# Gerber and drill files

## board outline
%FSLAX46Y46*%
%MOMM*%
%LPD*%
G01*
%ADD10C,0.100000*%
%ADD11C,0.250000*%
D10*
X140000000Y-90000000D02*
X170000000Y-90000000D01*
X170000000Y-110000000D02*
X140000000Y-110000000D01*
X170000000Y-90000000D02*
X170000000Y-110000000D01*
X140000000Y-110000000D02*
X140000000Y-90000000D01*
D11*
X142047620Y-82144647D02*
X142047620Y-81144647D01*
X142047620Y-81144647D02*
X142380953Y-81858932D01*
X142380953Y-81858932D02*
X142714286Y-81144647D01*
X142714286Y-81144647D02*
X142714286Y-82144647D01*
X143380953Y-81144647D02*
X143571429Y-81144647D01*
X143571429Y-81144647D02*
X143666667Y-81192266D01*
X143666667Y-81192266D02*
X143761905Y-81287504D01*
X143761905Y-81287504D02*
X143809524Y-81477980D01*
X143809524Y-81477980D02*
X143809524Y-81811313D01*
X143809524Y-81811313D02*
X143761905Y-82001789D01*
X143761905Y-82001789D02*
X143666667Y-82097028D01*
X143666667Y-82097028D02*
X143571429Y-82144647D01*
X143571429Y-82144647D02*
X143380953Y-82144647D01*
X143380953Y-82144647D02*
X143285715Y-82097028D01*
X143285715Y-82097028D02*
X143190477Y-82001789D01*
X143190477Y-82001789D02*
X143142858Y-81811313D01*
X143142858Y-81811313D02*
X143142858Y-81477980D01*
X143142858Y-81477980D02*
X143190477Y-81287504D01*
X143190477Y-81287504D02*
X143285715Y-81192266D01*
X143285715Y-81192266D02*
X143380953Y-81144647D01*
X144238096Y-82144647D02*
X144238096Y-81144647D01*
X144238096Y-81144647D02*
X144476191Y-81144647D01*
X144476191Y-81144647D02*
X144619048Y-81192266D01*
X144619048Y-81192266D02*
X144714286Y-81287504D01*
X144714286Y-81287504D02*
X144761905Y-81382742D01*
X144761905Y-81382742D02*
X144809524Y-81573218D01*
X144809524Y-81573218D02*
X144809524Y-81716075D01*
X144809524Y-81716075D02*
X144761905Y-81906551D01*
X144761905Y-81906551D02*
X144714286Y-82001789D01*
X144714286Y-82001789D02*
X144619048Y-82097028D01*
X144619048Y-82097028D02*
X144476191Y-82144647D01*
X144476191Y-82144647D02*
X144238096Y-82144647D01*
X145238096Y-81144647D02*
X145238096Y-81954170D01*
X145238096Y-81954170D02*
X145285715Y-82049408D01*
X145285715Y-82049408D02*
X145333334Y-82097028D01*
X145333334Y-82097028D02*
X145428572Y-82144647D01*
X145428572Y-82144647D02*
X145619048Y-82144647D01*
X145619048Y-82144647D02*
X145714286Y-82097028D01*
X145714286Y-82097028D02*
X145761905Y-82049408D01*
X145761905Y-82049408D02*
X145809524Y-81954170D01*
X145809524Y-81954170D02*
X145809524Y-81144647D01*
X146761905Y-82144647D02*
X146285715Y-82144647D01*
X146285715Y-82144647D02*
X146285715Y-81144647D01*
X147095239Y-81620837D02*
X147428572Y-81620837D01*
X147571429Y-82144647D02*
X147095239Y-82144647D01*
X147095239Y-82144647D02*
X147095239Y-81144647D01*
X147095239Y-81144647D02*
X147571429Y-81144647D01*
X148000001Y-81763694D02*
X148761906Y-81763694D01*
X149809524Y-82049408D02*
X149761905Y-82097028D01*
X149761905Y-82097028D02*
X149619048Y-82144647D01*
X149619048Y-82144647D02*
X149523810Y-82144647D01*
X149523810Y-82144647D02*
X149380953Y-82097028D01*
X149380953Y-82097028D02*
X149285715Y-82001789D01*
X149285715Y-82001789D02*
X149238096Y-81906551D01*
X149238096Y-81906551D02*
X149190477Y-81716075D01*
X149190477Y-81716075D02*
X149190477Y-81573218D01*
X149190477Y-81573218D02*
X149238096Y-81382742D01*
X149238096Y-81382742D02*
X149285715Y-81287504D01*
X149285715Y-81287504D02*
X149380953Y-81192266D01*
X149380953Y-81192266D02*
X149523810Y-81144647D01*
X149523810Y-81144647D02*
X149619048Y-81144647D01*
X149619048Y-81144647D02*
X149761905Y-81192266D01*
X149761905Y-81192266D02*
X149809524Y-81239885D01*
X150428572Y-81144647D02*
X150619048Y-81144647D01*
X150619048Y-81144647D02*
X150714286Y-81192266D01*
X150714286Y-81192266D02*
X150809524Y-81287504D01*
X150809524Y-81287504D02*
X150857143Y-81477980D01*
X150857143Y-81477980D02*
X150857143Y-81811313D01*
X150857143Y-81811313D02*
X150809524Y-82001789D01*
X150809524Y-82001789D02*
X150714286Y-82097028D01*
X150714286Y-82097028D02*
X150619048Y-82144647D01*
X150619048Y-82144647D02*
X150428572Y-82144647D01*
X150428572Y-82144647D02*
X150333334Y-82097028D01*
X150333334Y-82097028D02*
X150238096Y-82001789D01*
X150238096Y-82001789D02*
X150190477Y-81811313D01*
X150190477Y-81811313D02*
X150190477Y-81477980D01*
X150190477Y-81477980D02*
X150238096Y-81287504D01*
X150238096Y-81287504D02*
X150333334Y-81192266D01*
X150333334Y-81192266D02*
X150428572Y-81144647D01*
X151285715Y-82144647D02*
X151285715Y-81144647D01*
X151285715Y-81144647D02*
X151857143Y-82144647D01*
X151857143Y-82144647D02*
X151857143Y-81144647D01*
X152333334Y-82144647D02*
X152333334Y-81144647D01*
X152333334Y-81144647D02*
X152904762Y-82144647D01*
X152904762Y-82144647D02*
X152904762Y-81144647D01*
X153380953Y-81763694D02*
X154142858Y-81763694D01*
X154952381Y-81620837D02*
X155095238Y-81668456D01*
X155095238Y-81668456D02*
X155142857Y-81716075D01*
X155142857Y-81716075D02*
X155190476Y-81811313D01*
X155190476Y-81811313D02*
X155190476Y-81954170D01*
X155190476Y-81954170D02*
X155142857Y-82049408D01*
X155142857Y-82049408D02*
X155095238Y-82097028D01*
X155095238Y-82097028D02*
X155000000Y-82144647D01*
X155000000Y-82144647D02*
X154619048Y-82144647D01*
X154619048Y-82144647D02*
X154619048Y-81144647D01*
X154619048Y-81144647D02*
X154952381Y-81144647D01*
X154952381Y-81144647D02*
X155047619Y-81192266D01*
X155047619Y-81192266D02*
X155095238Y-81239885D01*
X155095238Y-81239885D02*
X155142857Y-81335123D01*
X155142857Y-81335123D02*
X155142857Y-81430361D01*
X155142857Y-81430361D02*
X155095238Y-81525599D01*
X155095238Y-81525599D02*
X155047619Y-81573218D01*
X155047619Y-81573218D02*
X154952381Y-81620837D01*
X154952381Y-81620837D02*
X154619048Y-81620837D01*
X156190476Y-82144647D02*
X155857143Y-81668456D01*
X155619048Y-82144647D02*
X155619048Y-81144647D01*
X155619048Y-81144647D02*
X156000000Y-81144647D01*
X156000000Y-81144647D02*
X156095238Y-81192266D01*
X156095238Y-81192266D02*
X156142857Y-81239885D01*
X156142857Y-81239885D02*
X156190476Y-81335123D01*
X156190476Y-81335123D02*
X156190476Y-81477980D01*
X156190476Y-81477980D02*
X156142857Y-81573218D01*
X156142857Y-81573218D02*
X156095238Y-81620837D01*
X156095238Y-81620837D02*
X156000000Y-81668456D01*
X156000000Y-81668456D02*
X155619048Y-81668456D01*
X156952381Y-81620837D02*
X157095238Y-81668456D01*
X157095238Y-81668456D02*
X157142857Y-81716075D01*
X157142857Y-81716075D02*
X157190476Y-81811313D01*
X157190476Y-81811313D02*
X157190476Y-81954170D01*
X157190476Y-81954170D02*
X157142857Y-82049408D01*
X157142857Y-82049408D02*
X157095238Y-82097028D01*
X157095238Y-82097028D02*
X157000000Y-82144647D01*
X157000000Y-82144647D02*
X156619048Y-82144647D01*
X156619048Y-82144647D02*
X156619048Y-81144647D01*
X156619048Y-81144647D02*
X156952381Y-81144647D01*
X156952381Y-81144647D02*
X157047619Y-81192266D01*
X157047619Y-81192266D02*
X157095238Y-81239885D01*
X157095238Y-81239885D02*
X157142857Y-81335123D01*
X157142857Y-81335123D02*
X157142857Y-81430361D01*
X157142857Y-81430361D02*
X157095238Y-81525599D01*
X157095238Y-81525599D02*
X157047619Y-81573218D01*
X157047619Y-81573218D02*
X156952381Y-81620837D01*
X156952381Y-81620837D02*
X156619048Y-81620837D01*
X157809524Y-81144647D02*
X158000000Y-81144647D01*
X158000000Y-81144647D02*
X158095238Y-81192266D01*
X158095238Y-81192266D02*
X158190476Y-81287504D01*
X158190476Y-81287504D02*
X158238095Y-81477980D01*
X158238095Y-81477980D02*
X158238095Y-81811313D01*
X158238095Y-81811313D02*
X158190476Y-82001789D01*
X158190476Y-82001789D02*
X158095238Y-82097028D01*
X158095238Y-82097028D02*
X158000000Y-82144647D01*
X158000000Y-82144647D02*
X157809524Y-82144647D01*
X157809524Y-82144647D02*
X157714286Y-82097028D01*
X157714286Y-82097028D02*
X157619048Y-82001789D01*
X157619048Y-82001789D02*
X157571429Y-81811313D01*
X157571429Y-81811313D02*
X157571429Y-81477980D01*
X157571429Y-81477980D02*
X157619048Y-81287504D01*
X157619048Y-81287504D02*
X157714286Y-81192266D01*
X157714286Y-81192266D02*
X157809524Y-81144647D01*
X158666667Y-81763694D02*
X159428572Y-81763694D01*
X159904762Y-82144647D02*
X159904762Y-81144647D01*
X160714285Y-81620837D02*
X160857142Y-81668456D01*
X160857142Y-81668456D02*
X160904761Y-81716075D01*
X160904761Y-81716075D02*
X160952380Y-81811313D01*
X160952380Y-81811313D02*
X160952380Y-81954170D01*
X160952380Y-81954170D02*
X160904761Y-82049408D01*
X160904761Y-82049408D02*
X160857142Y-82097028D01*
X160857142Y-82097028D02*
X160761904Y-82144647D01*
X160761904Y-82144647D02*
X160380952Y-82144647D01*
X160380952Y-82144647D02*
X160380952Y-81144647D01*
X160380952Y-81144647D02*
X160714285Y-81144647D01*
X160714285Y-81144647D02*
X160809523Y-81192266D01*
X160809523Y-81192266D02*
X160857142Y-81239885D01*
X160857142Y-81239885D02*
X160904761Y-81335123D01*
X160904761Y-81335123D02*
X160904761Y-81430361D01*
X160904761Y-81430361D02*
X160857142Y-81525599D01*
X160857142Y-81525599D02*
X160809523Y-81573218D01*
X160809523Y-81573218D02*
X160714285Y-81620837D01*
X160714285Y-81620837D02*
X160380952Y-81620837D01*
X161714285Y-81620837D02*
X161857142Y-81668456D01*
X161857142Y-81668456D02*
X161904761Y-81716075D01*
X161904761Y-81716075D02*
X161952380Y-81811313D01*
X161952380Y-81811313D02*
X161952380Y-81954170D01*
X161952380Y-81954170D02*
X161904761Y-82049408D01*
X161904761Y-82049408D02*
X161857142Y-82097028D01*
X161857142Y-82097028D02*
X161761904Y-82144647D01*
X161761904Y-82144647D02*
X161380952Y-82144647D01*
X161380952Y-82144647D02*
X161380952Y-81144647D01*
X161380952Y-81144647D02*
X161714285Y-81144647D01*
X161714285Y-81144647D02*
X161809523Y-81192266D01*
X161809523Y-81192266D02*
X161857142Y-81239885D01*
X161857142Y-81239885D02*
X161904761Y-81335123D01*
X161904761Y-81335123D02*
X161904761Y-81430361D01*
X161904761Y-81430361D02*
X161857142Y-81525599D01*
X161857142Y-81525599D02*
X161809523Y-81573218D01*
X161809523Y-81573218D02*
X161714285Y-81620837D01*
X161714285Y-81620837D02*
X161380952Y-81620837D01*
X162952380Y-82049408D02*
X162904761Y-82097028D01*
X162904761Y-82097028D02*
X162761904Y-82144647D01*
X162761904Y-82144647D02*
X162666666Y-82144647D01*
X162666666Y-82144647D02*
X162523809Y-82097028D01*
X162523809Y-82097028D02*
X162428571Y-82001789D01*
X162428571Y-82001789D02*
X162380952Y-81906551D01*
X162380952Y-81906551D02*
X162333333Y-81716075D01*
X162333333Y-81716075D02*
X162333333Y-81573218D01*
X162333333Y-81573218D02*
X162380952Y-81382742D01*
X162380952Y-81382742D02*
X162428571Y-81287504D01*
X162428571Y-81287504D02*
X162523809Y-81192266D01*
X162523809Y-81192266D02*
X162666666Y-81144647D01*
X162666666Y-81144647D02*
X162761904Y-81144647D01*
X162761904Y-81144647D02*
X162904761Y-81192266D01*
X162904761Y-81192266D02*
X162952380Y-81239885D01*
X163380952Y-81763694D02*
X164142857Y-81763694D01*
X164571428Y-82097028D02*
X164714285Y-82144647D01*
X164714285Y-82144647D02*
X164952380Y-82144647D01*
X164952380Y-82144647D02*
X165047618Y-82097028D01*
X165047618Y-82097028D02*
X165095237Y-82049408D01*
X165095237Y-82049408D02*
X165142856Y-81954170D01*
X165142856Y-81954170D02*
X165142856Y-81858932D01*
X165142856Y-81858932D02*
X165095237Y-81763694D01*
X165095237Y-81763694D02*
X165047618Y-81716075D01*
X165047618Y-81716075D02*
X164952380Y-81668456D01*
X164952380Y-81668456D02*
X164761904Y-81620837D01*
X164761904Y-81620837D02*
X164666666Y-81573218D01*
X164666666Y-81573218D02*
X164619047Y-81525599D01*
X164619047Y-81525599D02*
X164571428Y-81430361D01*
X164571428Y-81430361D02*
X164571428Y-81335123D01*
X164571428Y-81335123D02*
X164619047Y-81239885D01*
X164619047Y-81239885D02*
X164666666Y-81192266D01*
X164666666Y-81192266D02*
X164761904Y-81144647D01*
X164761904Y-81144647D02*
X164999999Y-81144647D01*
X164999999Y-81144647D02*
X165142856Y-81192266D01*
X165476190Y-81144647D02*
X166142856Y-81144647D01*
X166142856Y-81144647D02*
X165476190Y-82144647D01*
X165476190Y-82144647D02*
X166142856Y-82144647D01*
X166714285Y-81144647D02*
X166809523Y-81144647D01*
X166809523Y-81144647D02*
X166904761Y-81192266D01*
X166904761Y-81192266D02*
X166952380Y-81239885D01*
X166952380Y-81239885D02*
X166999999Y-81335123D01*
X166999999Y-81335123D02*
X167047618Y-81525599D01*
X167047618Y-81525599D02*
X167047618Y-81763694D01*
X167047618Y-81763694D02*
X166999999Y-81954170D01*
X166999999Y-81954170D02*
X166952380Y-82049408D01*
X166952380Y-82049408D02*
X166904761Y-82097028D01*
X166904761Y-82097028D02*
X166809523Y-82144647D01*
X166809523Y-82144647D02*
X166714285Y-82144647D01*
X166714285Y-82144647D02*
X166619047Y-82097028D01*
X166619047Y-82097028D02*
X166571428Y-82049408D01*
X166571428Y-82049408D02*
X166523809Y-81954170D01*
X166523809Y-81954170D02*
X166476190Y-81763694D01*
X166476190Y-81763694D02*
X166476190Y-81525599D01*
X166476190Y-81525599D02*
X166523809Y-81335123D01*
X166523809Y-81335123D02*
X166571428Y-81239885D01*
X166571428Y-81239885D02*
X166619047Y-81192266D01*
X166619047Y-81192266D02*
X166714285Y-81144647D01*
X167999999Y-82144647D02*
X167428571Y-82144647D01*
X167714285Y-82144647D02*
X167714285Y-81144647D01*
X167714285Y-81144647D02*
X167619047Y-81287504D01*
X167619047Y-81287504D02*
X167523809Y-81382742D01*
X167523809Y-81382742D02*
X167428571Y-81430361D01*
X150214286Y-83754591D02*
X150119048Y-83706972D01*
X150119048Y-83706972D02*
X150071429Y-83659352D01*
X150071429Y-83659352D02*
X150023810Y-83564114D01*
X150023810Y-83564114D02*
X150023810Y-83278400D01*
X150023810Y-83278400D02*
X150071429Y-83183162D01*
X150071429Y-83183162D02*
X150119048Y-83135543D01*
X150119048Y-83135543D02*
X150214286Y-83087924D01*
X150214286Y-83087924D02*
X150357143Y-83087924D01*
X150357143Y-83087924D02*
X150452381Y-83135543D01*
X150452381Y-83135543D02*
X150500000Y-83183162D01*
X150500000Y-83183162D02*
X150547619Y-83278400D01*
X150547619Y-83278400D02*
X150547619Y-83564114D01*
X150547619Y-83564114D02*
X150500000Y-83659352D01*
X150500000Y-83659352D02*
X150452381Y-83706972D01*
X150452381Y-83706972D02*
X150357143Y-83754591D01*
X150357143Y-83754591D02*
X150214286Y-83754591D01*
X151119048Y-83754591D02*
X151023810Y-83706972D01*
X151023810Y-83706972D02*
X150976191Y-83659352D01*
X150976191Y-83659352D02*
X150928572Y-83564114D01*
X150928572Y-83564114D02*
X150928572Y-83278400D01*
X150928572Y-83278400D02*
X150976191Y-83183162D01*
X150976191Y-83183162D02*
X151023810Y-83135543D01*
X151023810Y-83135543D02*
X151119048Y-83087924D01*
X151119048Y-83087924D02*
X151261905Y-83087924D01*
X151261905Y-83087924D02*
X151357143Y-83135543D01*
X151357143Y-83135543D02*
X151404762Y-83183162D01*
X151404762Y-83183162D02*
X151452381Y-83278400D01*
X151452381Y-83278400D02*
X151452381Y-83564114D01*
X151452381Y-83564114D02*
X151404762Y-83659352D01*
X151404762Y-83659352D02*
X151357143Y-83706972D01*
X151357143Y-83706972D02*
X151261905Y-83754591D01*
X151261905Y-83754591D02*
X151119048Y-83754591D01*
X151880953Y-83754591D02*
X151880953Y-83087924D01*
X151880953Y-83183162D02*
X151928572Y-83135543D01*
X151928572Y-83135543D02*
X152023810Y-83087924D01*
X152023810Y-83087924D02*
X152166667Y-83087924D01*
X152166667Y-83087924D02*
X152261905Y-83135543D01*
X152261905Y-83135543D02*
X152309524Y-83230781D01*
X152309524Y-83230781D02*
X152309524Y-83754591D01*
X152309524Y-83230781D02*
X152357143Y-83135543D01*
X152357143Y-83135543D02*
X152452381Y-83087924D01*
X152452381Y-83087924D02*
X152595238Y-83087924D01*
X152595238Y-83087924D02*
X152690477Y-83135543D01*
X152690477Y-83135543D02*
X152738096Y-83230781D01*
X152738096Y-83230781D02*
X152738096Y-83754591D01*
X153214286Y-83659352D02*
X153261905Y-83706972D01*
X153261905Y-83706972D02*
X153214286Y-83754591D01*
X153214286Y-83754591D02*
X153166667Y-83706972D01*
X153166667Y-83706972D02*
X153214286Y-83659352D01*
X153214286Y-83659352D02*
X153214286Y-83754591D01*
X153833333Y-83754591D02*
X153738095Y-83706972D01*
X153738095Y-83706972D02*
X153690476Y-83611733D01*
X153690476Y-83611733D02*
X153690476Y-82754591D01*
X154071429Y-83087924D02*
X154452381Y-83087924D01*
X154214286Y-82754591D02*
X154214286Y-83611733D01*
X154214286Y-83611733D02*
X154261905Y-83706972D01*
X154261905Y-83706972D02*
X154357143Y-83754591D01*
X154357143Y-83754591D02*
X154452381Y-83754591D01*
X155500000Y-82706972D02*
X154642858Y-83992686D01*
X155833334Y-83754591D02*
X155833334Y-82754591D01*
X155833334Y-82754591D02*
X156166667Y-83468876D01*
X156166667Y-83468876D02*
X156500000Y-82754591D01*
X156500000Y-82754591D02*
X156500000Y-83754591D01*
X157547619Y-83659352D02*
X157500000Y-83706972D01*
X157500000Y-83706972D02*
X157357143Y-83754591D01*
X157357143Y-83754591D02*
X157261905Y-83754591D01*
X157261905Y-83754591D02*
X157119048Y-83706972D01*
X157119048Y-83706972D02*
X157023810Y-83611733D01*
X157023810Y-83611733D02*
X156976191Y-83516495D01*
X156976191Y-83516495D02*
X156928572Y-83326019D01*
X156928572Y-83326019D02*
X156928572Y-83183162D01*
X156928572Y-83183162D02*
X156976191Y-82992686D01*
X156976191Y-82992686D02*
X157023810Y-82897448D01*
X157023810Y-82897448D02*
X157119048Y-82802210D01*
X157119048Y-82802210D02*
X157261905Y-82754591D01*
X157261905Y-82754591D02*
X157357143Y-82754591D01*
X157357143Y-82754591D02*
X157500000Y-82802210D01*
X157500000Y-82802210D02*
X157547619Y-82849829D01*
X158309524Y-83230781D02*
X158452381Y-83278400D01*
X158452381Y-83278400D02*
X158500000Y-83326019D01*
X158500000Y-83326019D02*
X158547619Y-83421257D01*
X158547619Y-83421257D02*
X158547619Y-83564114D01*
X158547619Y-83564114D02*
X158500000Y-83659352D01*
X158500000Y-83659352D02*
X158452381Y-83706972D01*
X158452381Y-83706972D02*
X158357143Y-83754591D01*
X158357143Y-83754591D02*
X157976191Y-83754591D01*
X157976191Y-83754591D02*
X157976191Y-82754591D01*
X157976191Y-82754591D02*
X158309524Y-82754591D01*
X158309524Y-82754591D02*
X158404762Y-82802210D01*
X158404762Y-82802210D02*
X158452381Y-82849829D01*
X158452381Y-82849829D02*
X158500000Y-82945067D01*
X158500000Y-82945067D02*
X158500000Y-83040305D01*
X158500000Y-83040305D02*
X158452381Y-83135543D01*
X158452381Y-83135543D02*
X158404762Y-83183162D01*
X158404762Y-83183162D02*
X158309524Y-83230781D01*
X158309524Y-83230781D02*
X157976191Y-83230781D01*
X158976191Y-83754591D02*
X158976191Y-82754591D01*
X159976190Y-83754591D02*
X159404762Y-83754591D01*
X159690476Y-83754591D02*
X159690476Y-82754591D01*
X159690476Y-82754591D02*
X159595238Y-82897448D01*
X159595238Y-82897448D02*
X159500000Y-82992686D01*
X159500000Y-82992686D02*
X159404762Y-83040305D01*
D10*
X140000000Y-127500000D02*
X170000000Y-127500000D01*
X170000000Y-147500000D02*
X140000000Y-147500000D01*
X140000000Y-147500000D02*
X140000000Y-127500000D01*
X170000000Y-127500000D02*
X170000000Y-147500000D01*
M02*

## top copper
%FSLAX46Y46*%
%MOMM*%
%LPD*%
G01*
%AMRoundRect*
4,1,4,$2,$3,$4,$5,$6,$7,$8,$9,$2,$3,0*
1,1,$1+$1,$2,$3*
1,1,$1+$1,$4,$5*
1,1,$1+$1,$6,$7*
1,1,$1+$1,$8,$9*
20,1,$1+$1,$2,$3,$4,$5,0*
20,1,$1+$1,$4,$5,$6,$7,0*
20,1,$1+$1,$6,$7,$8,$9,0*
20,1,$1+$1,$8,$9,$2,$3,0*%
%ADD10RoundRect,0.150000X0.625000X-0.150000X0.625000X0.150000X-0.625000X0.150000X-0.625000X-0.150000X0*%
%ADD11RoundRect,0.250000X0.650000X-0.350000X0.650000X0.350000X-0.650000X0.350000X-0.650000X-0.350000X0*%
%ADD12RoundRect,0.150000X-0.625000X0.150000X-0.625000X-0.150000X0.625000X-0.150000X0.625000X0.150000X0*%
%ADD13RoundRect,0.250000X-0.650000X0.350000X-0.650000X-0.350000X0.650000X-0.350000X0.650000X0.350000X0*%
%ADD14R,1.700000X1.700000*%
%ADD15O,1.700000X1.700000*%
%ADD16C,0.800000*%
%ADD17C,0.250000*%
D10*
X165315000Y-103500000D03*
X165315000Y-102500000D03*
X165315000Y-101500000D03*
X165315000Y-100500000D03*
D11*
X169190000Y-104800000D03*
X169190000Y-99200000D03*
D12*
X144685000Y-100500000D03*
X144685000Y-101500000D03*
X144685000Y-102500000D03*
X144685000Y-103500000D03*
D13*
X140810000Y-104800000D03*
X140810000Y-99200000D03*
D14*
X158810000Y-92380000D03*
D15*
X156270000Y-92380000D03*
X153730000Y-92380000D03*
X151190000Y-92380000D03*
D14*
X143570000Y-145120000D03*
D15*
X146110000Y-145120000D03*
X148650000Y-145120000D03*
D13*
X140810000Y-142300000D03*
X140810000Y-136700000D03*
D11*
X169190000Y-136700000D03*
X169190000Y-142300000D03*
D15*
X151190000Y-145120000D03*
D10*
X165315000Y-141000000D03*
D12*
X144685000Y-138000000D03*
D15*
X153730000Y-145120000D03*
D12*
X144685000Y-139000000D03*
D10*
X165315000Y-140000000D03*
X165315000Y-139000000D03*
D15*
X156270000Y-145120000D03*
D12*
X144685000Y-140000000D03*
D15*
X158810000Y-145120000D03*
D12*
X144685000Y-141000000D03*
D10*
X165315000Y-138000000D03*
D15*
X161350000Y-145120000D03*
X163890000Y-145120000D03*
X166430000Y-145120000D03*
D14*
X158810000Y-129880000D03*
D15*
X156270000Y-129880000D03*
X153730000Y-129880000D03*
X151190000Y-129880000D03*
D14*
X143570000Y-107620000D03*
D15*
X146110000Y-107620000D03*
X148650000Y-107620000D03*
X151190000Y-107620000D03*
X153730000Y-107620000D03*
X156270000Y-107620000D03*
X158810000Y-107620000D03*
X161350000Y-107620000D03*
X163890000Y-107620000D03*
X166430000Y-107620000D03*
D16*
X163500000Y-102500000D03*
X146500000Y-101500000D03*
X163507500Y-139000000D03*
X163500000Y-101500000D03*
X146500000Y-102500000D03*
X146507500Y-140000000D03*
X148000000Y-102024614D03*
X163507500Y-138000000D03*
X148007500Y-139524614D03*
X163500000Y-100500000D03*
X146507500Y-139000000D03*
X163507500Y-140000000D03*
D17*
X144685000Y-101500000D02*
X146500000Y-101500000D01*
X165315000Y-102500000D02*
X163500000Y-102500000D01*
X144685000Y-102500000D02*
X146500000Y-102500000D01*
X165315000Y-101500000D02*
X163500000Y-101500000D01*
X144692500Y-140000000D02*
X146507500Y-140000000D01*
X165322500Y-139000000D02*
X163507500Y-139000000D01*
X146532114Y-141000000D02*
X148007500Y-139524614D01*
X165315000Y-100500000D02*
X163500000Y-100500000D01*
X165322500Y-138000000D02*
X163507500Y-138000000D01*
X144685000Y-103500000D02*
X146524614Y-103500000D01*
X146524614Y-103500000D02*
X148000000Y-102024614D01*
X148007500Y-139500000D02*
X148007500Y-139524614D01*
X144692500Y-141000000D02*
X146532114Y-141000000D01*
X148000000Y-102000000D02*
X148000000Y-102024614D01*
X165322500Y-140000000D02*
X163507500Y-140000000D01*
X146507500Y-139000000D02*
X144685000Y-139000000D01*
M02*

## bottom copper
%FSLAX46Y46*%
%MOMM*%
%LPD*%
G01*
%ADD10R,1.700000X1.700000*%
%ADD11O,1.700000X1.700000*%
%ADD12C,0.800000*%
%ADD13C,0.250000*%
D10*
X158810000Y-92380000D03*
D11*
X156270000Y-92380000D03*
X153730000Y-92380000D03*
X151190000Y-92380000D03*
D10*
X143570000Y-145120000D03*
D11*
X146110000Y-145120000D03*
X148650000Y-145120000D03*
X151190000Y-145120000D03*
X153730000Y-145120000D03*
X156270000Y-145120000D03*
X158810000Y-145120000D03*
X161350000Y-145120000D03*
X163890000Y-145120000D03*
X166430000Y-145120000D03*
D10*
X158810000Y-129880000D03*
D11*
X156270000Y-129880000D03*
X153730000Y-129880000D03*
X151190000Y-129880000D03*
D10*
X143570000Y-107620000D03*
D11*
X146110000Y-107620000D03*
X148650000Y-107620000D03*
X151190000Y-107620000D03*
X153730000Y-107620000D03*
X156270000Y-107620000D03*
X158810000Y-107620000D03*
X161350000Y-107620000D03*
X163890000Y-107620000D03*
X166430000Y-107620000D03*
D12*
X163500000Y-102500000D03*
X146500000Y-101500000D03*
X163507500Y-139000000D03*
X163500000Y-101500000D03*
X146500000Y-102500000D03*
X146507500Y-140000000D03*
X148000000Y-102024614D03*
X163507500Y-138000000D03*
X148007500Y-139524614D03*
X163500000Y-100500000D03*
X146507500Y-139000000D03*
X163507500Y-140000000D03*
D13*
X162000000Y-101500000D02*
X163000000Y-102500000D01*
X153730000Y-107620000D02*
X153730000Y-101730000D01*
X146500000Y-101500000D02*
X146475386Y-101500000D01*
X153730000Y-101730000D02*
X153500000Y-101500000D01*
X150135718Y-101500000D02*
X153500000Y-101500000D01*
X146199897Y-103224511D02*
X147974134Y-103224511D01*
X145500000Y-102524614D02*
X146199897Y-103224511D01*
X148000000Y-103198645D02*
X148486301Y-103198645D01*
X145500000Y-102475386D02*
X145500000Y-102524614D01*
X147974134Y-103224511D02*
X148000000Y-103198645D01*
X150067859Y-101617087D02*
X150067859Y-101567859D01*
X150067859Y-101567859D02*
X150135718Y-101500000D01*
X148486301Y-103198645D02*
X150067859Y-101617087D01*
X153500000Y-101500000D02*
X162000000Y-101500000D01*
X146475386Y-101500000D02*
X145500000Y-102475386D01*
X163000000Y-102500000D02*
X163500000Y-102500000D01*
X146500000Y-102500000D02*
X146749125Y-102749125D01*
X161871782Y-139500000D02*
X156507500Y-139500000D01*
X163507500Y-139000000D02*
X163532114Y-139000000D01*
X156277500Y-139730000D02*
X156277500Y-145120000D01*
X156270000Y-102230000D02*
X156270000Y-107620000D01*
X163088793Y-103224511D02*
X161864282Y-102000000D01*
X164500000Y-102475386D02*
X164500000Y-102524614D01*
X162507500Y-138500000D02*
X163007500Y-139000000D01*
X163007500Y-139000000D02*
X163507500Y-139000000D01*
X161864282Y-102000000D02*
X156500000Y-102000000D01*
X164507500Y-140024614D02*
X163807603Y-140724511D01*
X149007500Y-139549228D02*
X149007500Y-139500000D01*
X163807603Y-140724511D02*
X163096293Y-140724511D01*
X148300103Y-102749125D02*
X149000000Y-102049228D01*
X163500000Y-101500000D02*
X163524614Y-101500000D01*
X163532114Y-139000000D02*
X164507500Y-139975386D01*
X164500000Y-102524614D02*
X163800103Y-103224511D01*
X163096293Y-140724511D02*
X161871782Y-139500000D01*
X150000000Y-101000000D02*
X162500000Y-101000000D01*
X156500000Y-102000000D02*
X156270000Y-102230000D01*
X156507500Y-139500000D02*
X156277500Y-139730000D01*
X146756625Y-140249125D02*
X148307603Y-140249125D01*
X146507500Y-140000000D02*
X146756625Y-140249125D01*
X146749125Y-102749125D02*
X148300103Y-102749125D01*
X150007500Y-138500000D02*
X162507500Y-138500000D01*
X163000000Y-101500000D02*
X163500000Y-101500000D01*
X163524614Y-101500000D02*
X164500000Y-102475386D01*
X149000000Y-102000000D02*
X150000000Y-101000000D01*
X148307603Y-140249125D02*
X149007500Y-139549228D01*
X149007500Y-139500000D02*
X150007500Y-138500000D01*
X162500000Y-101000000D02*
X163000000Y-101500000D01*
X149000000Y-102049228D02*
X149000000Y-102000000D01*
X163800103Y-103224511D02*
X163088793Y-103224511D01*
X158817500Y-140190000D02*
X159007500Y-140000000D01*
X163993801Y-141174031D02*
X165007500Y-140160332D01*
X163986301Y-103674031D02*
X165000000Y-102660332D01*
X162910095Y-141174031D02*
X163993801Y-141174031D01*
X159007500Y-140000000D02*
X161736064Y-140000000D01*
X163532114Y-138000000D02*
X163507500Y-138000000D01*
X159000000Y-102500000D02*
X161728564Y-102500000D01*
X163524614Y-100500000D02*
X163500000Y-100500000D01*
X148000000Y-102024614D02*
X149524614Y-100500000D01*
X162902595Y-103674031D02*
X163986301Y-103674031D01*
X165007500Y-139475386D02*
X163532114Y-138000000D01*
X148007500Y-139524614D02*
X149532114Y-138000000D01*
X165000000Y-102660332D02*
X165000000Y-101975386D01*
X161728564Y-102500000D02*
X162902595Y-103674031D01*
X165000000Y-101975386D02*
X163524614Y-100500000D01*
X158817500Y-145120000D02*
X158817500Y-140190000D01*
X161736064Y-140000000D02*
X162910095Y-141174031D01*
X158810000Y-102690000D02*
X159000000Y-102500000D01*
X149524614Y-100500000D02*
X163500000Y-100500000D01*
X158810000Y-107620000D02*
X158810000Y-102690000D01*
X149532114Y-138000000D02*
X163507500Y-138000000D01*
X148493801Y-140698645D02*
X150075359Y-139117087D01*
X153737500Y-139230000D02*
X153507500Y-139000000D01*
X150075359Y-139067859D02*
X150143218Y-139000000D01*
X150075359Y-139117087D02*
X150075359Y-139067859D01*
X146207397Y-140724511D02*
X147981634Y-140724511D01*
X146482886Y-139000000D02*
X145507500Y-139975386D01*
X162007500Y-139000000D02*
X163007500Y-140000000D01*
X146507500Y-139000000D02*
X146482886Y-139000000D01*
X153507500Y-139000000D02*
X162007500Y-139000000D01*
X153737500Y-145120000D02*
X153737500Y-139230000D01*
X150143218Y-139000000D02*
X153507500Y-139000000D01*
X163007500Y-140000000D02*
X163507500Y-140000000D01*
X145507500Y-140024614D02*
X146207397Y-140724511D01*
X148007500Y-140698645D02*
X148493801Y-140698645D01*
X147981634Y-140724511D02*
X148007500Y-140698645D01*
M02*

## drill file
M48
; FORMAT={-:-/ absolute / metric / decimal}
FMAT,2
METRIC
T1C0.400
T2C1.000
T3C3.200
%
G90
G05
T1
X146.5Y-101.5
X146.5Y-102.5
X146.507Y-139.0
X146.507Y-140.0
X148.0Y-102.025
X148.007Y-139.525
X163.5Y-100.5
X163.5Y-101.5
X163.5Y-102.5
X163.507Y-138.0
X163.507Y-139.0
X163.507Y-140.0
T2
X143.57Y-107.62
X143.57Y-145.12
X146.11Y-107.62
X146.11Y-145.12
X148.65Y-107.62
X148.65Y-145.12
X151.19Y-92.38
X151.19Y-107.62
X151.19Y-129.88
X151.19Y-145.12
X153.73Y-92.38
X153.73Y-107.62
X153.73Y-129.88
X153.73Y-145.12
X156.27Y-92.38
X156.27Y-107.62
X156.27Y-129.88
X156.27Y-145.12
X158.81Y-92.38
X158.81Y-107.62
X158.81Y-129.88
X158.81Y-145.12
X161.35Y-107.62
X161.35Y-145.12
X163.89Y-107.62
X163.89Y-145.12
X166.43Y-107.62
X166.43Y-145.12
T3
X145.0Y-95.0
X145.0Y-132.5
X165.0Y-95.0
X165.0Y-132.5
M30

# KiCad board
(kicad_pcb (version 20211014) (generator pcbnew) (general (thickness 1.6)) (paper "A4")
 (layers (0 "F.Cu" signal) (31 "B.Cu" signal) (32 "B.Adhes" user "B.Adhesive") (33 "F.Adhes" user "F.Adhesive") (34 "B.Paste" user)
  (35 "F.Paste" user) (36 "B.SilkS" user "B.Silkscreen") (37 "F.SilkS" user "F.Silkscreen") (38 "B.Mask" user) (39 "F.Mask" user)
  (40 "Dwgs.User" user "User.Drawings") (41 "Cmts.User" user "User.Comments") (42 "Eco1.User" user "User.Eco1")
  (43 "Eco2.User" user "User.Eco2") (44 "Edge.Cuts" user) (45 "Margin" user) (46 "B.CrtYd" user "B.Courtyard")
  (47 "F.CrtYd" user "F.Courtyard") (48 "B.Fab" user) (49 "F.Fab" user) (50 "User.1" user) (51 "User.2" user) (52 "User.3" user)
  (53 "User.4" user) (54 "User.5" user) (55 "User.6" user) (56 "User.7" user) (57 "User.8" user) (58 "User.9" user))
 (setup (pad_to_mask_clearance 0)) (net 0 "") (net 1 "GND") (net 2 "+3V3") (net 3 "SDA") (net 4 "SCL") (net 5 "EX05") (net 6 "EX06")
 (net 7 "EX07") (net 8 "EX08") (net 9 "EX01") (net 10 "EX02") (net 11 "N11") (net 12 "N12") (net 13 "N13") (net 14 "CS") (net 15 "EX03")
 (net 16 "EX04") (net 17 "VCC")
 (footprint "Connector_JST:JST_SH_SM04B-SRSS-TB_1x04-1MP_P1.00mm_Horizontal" (layer "F.Cu") (at 167.315 102 90)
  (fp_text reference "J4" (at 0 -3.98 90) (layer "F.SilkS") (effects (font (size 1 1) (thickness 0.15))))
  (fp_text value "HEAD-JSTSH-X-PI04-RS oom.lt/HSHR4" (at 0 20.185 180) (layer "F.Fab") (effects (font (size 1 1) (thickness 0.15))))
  (pad "1" smd roundrect (at -1.5 -2 90) (size 0.6 1.55) (layers "F.Cu" "F.Paste" "F.Mask") (roundrect_rratio 0.25) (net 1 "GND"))
  (pad "2" smd roundrect (at -0.5 -2 90) (size 0.6 1.55) (layers "F.Cu" "F.Paste" "F.Mask") (roundrect_rratio 0.25) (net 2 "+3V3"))
  (pad "3" smd roundrect (at 0.5 -2 90) (size 0.6 1.55) (layers "F.Cu" "F.Paste" "F.Mask") (roundrect_rratio 0.25) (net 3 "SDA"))
  (pad "4" smd roundrect (at 1.5 -2 90) (size 0.6 1.55) (layers "F.Cu" "F.Paste" "F.Mask") (roundrect_rratio 0.25) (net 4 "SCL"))
  (pad "MP" smd roundrect (at -2.8 1.875 90) (size 1.2 1.8) (layers "F.Cu" "F.Paste" "F.Mask") (roundrect_rratio 0.208333) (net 1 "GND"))
  (pad "MP" smd roundrect (at 2.8 1.875 90) (size 1.2 1.8) (layers "F.Cu" "F.Paste" "F.Mask") (roundrect_rratio 0.208333) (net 1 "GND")))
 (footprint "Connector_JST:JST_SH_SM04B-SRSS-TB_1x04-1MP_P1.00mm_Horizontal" (layer "F.Cu") (at 142.685 102 -90)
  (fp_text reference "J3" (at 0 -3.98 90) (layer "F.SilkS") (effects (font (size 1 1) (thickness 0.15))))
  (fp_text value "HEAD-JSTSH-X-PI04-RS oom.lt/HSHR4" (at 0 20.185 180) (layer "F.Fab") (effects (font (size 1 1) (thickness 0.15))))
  (pad "1" smd roundrect (at -1.5 -2 270) (size 0.6 1.55) (layers "F.Cu" "F.Paste" "F.Mask") (roundrect_rratio 0.25) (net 1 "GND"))
  (pad "2" smd roundrect (at -0.5 -2 270) (size 0.6 1.55) (layers "F.Cu" "F.Paste" "F.Mask") (roundrect_rratio 0.25) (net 2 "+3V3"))
  (pad "3" smd roundrect (at 0.5 -2 270) (size 0.6 1.55) (layers "F.Cu" "F.Paste" "F.Mask") (roundrect_rratio 0.25) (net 3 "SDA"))
  (pad "4" smd roundrect (at 1.5 -2 270) (size 0.6 1.55) (layers "F.Cu" "F.Paste" "F.Mask") (roundrect_rratio 0.25) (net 4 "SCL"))
  (pad "MP" smd roundrect (at 2.8 1.875 270) (size 1.2 1.8) (layers "F.Cu" "F.Paste" "F.Mask") (roundrect_rratio 0.208333) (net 1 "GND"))
  (pad "MP" smd roundrect (at -2.8 1.875 270) (size 1.2 1.8) (layers "F.Cu" "F.Paste" "F.Mask") (roundrect_rratio 0.208333) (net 1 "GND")))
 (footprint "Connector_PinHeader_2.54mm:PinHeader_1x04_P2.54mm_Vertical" (layer "F.Cu") (at 158.81 92.38 -90)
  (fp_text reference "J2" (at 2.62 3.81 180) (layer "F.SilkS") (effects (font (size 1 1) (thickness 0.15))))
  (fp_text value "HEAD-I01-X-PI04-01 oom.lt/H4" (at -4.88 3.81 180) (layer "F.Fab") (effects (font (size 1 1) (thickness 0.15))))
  (pad "1" thru_hole rect (at 0 0 270) (size 1.7 1.7) (drill 1) (layers *.Cu *.Mask) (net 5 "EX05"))
  (pad "2" thru_hole oval (at 0 2.54 270) (size 1.7 1.7) (drill 1) (layers *.Cu *.Mask) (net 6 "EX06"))
  (pad "3" thru_hole oval (at 0 5.08 270) (size 1.7 1.7) (drill 1) (layers *.Cu *.Mask) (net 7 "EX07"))
  (pad "4" thru_hole oval (at 0 7.62 270) (size 1.7 1.7) (drill 1) (layers *.Cu *.Mask) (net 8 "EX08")))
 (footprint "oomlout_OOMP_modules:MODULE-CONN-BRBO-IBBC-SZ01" (layer "F.Cu") (at 155 137.5)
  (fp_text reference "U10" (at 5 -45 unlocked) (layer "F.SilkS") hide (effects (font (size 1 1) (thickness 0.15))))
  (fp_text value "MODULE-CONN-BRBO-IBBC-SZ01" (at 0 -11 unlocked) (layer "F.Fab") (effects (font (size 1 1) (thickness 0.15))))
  (fp_line (start -15 -10) (end 15 -10) (layer "Edge.Cuts") (width 0.1))
  (fp_line (start 15 10) (end -15 10) (layer "Edge.Cuts") (width 0.1))
  (fp_line (start -15 10) (end -15 -10) (layer "Edge.Cuts") (width 0.1))
  (fp_line (start 15 -10) (end 15 10) (layer "Edge.Cuts") (width 0.1))
  (pad "" np_thru_hole circle (at 10 -5) (size 3.2 3.2) (drill 3.2) (layers *.Cu *.Mask))
  (pad "" np_thru_hole circle (at -10 -5) (size 3.2 3.2) (drill 3.2) (layers *.Cu *.Mask))
  (pad "1" thru_hole rect (at -11.43 7.62 90) (size 1.7 1.7) (drill 1) (layers *.Cu *.Mask) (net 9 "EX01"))
  (pad "2" thru_hole oval (at -8.89 7.62 90) (size 1.7 1.7) (drill 1) (layers *.Cu *.Mask) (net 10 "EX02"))
  (pad "3" thru_hole oval (at -6.35 7.62 90) (size 1.7 1.7) (drill 1) (layers *.Cu *.Mask) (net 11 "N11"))
  (pad "4" smd roundrect (at -14.19 4.8 270) (size 1.2 1.8) (layers "F.Cu" "F.Paste" "F.Mask") (roundrect_rratio 0.208333) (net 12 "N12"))
  (pad "4" smd roundrect (at -14.19 -0.8 270) (size 1.2 1.8) (layers "F.Cu" "F.Paste" "F.Mask") (roundrect_rratio 0.208333) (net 12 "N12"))
  (pad "4" smd roundrect (at 14.19 -0.8 90) (size 1.2 1.8) (layers "F.Cu" "F.Paste" "F.Mask") (roundrect_rratio 0.208333) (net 12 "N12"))
  (pad "4" smd roundrect (at 14.19 4.8 90) (size 1.2 1.8) (layers "F.Cu" "F.Paste" "F.Mask") (roundrect_rratio 0.208333) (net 12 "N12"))
  (pad "4" thru_hole oval (at -3.81 7.62 90) (size 1.7 1.7) (drill 1) (layers *.Cu *.Mask) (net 12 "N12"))
  (pad "4" smd roundrect (at 10.315 3.5 90) (size 0.6 1.55) (layers "F.Cu" "F.Paste" "F.Mask") (roundrect_rratio 0.25) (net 12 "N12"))
  (pad "4" smd roundrect (at -10.315 0.5 270) (size 0.6 1.55) (layers "F.Cu" "F.Paste" "F.Mask") (roundrect_rratio 0.25) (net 12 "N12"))
  (pad "5" thru_hole oval (at -1.27 7.62 90) (size 1.7 1.7) (drill 1) (layers *.Cu *.Mask) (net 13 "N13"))
  (pad "5" smd roundrect (at -10.315 1.5 270) (size 0.6 1.55) (layers "F.Cu" "F.Paste" "F.Mask") (roundrect_rratio 0.25) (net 13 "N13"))
  (pad "5" smd roundrect (at 10.315 2.5 90) (size 0.6 1.55) (layers "F.Cu" "F.Paste" "F.Mask") (roundrect_rratio 0.25) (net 13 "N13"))
  (pad "6" smd roundrect (at 10.315 1.5 90) (size 0.6 1.55) (layers "F.Cu" "F.Paste" "F.Mask") (roundrect_rratio 0.25) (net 3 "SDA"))
  (pad "6" thru_hole oval (at 1.27 7.62 90) (size 1.7 1.7) (drill 1) (layers *.Cu *.Mask) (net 3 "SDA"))
  (pad "6" smd roundrect (at -10.315 2.5 270) (size 0.6 1.55) (layers "F.Cu" "F.Paste" "F.Mask") (roundrect_rratio 0.25) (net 3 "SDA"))
  (pad "7" thru_hole oval (at 3.81 7.62 90) (size 1.7 1.7) (drill 1) (layers *.Cu *.Mask) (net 4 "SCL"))
  (pad "7" smd roundrect (at -10.315 3.5 270) (size 0.6 1.55) (layers "F.Cu" "F.Paste" "F.Mask") (roundrect_rratio 0.25) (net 4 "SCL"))
  (pad "7" smd roundrect (at 10.315 0.5 90) (size 0.6 1.55) (layers "F.Cu" "F.Paste" "F.Mask") (roundrect_rratio 0.25) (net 4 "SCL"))
  (pad "8" thru_hole oval (at 6.35 7.62 90) (size 1.7 1.7) (drill 1) (layers *.Cu *.Mask) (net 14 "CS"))
  (pad "9" thru_hole oval (at 8.89 7.62 90) (size 1.7 1.7) (drill 1) (layers *.Cu *.Mask) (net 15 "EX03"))
  (pad "10" thru_hole oval (at 11.43 7.62 90) (size 1.7 1.7) (drill 1) (layers *.Cu *.Mask) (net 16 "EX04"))
  (pad "11" thru_hole rect (at 3.81 -7.62 270) (size 1.7 1.7) (drill 1) (layers *.Cu *.Mask) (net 5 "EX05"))
  (pad "12" thru_hole oval (at 1.27 -7.62 270) (size 1.7 1.7) (drill 1) (layers *.Cu *.Mask) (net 6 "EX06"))
  (pad "13" thru_hole oval (at -1.27 -7.62 270) (size 1.7 1.7) (drill 1) (layers *.Cu *.Mask) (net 7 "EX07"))
  (pad "14" thru_hole oval (at -3.81 -7.62 270) (size 1.7 1.7) (drill 1) (layers *.Cu *.Mask) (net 8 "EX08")))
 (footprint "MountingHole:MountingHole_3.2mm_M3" (layer "F.Cu") (at 145 95)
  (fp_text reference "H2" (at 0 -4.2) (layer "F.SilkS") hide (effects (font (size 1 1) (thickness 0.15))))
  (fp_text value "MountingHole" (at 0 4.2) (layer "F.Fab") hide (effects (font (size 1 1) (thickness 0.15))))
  (pad "" np_thru_hole circle (at 0 0) (size 3.2 3.2) (drill 3.2) (layers *.Cu *.Mask)))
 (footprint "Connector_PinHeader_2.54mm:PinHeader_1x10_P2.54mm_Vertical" (layer "F.Cu") (at 143.57 107.62 90)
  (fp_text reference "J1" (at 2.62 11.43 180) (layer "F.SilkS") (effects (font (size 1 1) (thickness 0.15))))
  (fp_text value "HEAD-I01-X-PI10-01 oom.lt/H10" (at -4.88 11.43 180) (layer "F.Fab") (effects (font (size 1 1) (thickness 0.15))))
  (pad "1" thru_hole rect (at 0 0 90) (size 1.7 1.7) (drill 1) (layers *.Cu *.Mask) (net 9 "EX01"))
  (pad "2" thru_hole oval (at 0 2.54 90) (size 1.7 1.7) (drill 1) (layers *.Cu *.Mask) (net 10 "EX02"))
  (pad "3" thru_hole oval (at 0 5.08 90) (size 1.7 1.7) (drill 1) (layers *.Cu *.Mask) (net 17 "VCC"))
  (pad "4" thru_hole oval (at 0 7.62 90) (size 1.7 1.7) (drill 1) (layers *.Cu *.Mask) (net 1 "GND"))
  (pad "5" thru_hole oval (at 0 10.16 90) (size 1.7 1.7) (drill 1) (layers *.Cu *.Mask) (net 2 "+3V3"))
  (pad "6" thru_hole oval (at 0 12.7 90) (size 1.7 1.7) (drill 1) (layers *.Cu *.Mask) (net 3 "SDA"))
  (pad "7" thru_hole oval (at 0 15.24 90) (size 1.7 1.7) (drill 1) (layers *.Cu *.Mask) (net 4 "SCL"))
  (pad "8" thru_hole oval (at 0 17.78 90) (size 1.7 1.7) (drill 1) (layers *.Cu *.Mask) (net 14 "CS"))
  (pad "9" thru_hole oval (at 0 20.32 90) (size 1.7 1.7) (drill 1) (layers *.Cu *.Mask) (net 15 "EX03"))
  (pad "10" thru_hole oval (at 0 22.86 90) (size 1.7 1.7) (drill 1) (layers *.Cu *.Mask) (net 16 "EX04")))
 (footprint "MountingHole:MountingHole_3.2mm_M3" (layer "F.Cu") (at 165 95)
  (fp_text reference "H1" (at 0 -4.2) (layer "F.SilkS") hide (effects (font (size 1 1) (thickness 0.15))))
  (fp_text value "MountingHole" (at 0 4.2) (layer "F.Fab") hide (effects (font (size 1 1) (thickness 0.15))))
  (pad "" np_thru_hole circle (at 0 0) (size 3.2 3.2) (drill 3.2) (layers *.Cu *.Mask)))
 (gr_line (start 140 90) (end 170 90) (layer "Edge.Cuts") (width 0.1))
 (gr_line (start 170 110) (end 140 110) (layer "Edge.Cuts") (width 0.1))
 (gr_line (start 170 90) (end 170 110) (layer "Edge.Cuts") (width 0.1))
 (gr_line (start 140 110) (end 140 90) (layer "Edge.Cuts") (width 0.1))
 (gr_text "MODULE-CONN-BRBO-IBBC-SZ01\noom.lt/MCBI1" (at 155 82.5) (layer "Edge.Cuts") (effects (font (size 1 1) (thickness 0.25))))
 (segment (start 144.685 101.5) (end 146.5 101.5) (width 0.25) (layer "F.Cu") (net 2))
 (segment (start 165.315 102.5) (end 163.5 102.5) (width 0.25) (layer "F.Cu") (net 2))
 (via (at 163.5 102.5) (size 0.8) (drill 0.4) (layers "F.Cu" "B.Cu") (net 2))
 (via (at 146.5 101.5) (size 0.8) (drill 0.4) (layers "F.Cu" "B.Cu") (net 2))
 (segment (start 162 101.5) (end 163 102.5) (width 0.25) (layer "B.Cu") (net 2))
 (segment (start 153.73 107.62) (end 153.73 101.73) (width 0.25) (layer "B.Cu") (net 2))
 (segment (start 146.5 101.5) (end 146.475386 101.5) (width 0.25) (layer "B.Cu") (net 2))
 (segment (start 153.73 101.73) (end 153.5 101.5) (width 0.25) (layer "B.Cu") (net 2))
 (segment (start 150.135718 101.5) (end 153.5 101.5) (width 0.25) (layer "B.Cu") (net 2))
 (segment (start 146.199897 103.224511) (end 147.974134 103.224511) (width 0.25) (layer "B.Cu") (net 2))
 (segment (start 145.5 102.524614) (end 146.199897 103.224511) (width 0.25) (layer "B.Cu") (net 2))
 (segment (start 148 103.198645) (end 148.486301 103.198645) (width 0.25) (layer "B.Cu") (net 2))
 (segment (start 145.5 102.475386) (end 145.5 102.524614) (width 0.25) (layer "B.Cu") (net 2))
 (segment (start 147.974134 103.224511) (end 148 103.198645) (width 0.25) (layer "B.Cu") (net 2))
 (segment (start 150.067859 101.617087) (end 150.067859 101.567859) (width 0.25) (layer "B.Cu") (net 2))
 (segment (start 150.067859 101.567859) (end 150.135718 101.5) (width 0.25) (layer "B.Cu") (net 2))
 (segment (start 148.486301 103.198645) (end 150.067859 101.617087) (width 0.25) (layer "B.Cu") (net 2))
 (segment (start 153.5 101.5) (end 162 101.5) (width 0.25) (layer "B.Cu") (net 2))
 (segment (start 146.475386 101.5) (end 145.5 102.475386) (width 0.25) (layer "B.Cu") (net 2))
 (segment (start 163 102.5) (end 163.5 102.5) (width 0.25) (layer "B.Cu") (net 2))
 (segment (start 144.685 102.5) (end 146.5 102.5) (width 0.25) (layer "F.Cu") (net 3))
 (segment (start 165.315 101.5) (end 163.5 101.5) (width 0.25) (layer "F.Cu") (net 3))
 (segment (start 144.6925 140) (end 146.5075 140) (width 0.25) (layer "F.Cu") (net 3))
 (segment (start 165.3225 139) (end 163.5075 139) (width 0.25) (layer "F.Cu") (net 3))
 (via (at 163.5075 139) (size 0.8) (drill 0.4) (layers "F.Cu" "B.Cu") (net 3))
 (via (at 163.5 101.5) (size 0.8) (drill 0.4) (layers "F.Cu" "B.Cu") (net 3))
 (via (at 146.5 102.5) (size 0.8) (drill 0.4) (layers "F.Cu" "B.Cu") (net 3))
 (via (at 146.5075 140) (size 0.8) (drill 0.4) (layers "F.Cu" "B.Cu") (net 3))
 (segment (start 146.5 102.5) (end 146.749125 102.749125) (width 0.25) (layer "B.Cu") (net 3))
 (segment (start 161.871782 139.5) (end 156.5075 139.5) (width 0.25) (layer "B.Cu") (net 3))
 (segment (start 163.5075 139) (end 163.532114 139) (width 0.25) (layer "B.Cu") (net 3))
 (segment (start 156.2775 139.73) (end 156.2775 145.12) (width 0.25) (layer "B.Cu") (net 3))
 (segment (start 156.27 102.23) (end 156.27 107.62) (width 0.25) (layer "B.Cu") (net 3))
 (segment (start 163.088793 103.224511) (end 161.864282 102) (width 0.25) (layer "B.Cu") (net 3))
 (segment (start 164.5 102.475386) (end 164.5 102.524614) (width 0.25) (layer "B.Cu") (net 3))
 (segment (start 162.5075 138.5) (end 163.0075 139) (width 0.25) (layer "B.Cu") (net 3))
 (segment (start 163.0075 139) (end 163.5075 139) (width 0.25) (layer "B.Cu") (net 3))
 (segment (start 161.864282 102) (end 156.5 102) (width 0.25) (layer "B.Cu") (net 3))
 (segment (start 164.5075 140.024614) (end 163.807603 140.724511) (width 0.25) (layer "B.Cu") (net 3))
 (segment (start 149.0075 139.549228) (end 149.0075 139.5) (width 0.25) (layer "B.Cu") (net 3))
 (segment (start 163.807603 140.724511) (end 163.096293 140.724511) (width 0.25) (layer "B.Cu") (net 3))
 (segment (start 148.300103 102.749125) (end 149 102.049228) (width 0.25) (layer "B.Cu") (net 3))
 (segment (start 163.5 101.5) (end 163.524614 101.5) (width 0.25) (layer "B.Cu") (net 3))
 (segment (start 163.532114 139) (end 164.5075 139.975386) (width 0.25) (layer "B.Cu") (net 3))
 (segment (start 164.5 102.524614) (end 163.800103 103.224511) (width 0.25) (layer "B.Cu") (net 3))
 (segment (start 163.096293 140.724511) (end 161.871782 139.5) (width 0.25) (layer "B.Cu") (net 3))
 (segment (start 150 101) (end 162.5 101) (width 0.25) (layer "B.Cu") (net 3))
 (segment (start 156.5 102) (end 156.27 102.23) (width 0.25) (layer "B.Cu") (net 3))
 (segment (start 156.5075 139.5) (end 156.2775 139.73) (width 0.25) (layer "B.Cu") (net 3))
 (segment (start 146.756625 140.249125) (end 148.307603 140.249125) (width 0.25) (layer "B.Cu") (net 3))
 (segment (start 146.5075 140) (end 146.756625 140.249125) (width 0.25) (layer "B.Cu") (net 3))
 (segment (start 146.749125 102.749125) (end 148.300103 102.749125) (width 0.25) (layer "B.Cu") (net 3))
 (segment (start 150.0075 138.5) (end 162.5075 138.5) (width 0.25) (layer "B.Cu") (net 3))
 (segment (start 163 101.5) (end 163.5 101.5) (width 0.25) (layer "B.Cu") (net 3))
 (segment (start 163.524614 101.5) (end 164.5 102.475386) (width 0.25) (layer "B.Cu") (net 3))
 (segment (start 149 102) (end 150 101) (width 0.25) (layer "B.Cu") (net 3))
 (segment (start 148.307603 140.249125) (end 149.0075 139.549228) (width 0.25) (layer "B.Cu") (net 3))
 (segment (start 149.0075 139.5) (end 150.0075 138.5) (width 0.25) (layer "B.Cu") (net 3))
 (segment (start 162.5 101) (end 163 101.5) (width 0.25) (layer "B.Cu") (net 3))
 (segment (start 149 102.049228) (end 149 102) (width 0.25) (layer "B.Cu") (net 3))
 (segment (start 163.800103 103.224511) (end 163.088793 103.224511) (width 0.25) (layer "B.Cu") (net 3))
 (segment (start 146.532114 141) (end 148.0075 139.524614) (width 0.25) (layer "F.Cu") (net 4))
 (segment (start 165.315 100.5) (end 163.5 100.5) (width 0.25) (layer "F.Cu") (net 4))
 (segment (start 165.3225 138) (end 163.5075 138) (width 0.25) (layer "F.Cu") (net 4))
 (segment (start 144.685 103.5) (end 146.524614 103.5) (width 0.25) (layer "F.Cu") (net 4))
 (segment (start 146.524614 103.5) (end 148 102.024614) (width 0.25) (layer "F.Cu") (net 4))
 (segment (start 148.0075 139.5) (end 148.0075 139.524614) (width 0.25) (layer "F.Cu") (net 4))
 (segment (start 144.6925 141) (end 146.532114 141) (width 0.25) (layer "F.Cu") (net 4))
 (segment (start 148 102) (end 148 102.024614) (width 0.25) (layer "F.Cu") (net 4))
 (via (at 148 102.024614) (size 0.8) (drill 0.4) (layers "F.Cu" "B.Cu") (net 4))
 (via (at 163.5075 138) (size 0.8) (drill 0.4) (layers "F.Cu" "B.Cu") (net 4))
 (via (at 148.0075 139.524614) (size 0.8) (drill 0.4) (layers "F.Cu" "B.Cu") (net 4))
 (via (at 163.5 100.5) (size 0.8) (drill 0.4) (layers "F.Cu" "B.Cu") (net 4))
 (segment (start 158.8175 140.19) (end 159.0075 140) (width 0.25) (layer "B.Cu") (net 4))
 (segment (start 163.993801 141.174031) (end 165.0075 140.160332) (width 0.25) (layer "B.Cu") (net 4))
 (segment (start 163.986301 103.674031) (end 165 102.660332) (width 0.25) (layer "B.Cu") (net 4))
 (segment (start 162.910095 141.174031) (end 163.993801 141.174031) (width 0.25) (layer "B.Cu") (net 4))
 (segment (start 159.0075 140) (end 161.736064 140) (width 0.25) (layer "B.Cu") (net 4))
 (segment (start 163.532114 138) (end 163.5075 138) (width 0.25) (layer "B.Cu") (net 4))
 (segment (start 159 102.5) (end 161.728564 102.5) (width 0.25) (layer "B.Cu") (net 4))
 (segment (start 163.524614 100.5) (end 163.5 100.5) (width 0.25) (layer "B.Cu") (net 4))
 (segment (start 148 102.024614) (end 149.524614 100.5) (width 0.25) (layer "B.Cu") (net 4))
 (segment (start 162.902595 103.674031) (end 163.986301 103.674031) (width 0.25) (layer "B.Cu") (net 4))
 (segment (start 165.0075 139.475386) (end 163.532114 138) (width 0.25) (layer "B.Cu") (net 4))
 (segment (start 148.0075 139.524614) (end 149.532114 138) (width 0.25) (layer "B.Cu") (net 4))
 (segment (start 165 102.660332) (end 165 101.975386) (width 0.25) (layer "B.Cu") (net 4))
 (segment (start 161.728564 102.5) (end 162.902595 103.674031) (width 0.25) (layer "B.Cu") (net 4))
 (segment (start 165 101.975386) (end 163.524614 100.5) (width 0.25) (layer "B.Cu") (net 4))
 (segment (start 158.8175 145.12) (end 158.8175 140.19) (width 0.25) (layer "B.Cu") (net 4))
 (segment (start 161.736064 140) (end 162.910095 141.174031) (width 0.25) (layer "B.Cu") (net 4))
 (segment (start 158.81 102.69) (end 159 102.5) (width 0.25) (layer "B.Cu") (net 4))
 (segment (start 149.524614 100.5) (end 163.5 100.5) (width 0.25) (layer "B.Cu") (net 4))
 (segment (start 158.81 107.62) (end 158.81 102.69) (width 0.25) (layer "B.Cu") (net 4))
 (segment (start 149.532114 138) (end 163.5075 138) (width 0.25) (layer "B.Cu") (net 4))
 (segment (start 165.3225 140) (end 163.5075 140) (width 0.25) (layer "F.Cu") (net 13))
 (segment (start 146.5075 139) (end 144.685 139) (width 0.25) (layer "F.Cu") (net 13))
 (via (at 146.5075 139) (size 0.8) (drill 0.4) (layers "F.Cu" "B.Cu") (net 13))
 (via (at 163.5075 140) (size 0.8) (drill 0.4) (layers "F.Cu" "B.Cu") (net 13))
 (segment (start 148.493801 140.698645) (end 150.075359 139.117087) (width 0.25) (layer "B.Cu") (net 13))
 (segment (start 153.7375 139.23) (end 153.5075 139) (width 0.25) (layer "B.Cu") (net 13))
 (segment (start 150.075359 139.067859) (end 150.143218 139) (width 0.25) (layer "B.Cu") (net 13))
 (segment (start 150.075359 139.117087) (end 150.075359 139.067859) (width 0.25) (layer "B.Cu") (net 13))
 (segment (start 146.207397 140.724511) (end 147.981634 140.724511) (width 0.25) (layer "B.Cu") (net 13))
 (segment (start 146.482886 139) (end 145.5075 139.975386) (width 0.25) (layer "B.Cu") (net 13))
 (segment (start 162.0075 139) (end 163.0075 140) (width 0.25) (layer "B.Cu") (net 13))
 (segment (start 146.5075 139) (end 146.482886 139) (width 0.25) (layer "B.Cu") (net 13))
 (segment (start 153.5075 139) (end 162.0075 139) (width 0.25) (layer "B.Cu") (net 13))
 (segment (start 153.7375 145.12) (end 153.7375 139.23) (width 0.25) (layer "B.Cu") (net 13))
 (segment (start 150.143218 139) (end 153.5075 139) (width 0.25) (layer "B.Cu") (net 13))
 (segment (start 163.0075 140) (end 163.5075 140) (width 0.25) (layer "B.Cu") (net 13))
 (segment (start 145.5075 140.024614) (end 146.207397 140.724511) (width 0.25) (layer "B.Cu") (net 13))
 (segment (start 148.0075 140.698645) (end 148.493801 140.698645) (width 0.25) (layer "B.Cu") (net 13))
 (segment (start 147.981634 140.724511) (end 148.0075 140.698645) (width 0.25) (layer "B.Cu") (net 13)))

